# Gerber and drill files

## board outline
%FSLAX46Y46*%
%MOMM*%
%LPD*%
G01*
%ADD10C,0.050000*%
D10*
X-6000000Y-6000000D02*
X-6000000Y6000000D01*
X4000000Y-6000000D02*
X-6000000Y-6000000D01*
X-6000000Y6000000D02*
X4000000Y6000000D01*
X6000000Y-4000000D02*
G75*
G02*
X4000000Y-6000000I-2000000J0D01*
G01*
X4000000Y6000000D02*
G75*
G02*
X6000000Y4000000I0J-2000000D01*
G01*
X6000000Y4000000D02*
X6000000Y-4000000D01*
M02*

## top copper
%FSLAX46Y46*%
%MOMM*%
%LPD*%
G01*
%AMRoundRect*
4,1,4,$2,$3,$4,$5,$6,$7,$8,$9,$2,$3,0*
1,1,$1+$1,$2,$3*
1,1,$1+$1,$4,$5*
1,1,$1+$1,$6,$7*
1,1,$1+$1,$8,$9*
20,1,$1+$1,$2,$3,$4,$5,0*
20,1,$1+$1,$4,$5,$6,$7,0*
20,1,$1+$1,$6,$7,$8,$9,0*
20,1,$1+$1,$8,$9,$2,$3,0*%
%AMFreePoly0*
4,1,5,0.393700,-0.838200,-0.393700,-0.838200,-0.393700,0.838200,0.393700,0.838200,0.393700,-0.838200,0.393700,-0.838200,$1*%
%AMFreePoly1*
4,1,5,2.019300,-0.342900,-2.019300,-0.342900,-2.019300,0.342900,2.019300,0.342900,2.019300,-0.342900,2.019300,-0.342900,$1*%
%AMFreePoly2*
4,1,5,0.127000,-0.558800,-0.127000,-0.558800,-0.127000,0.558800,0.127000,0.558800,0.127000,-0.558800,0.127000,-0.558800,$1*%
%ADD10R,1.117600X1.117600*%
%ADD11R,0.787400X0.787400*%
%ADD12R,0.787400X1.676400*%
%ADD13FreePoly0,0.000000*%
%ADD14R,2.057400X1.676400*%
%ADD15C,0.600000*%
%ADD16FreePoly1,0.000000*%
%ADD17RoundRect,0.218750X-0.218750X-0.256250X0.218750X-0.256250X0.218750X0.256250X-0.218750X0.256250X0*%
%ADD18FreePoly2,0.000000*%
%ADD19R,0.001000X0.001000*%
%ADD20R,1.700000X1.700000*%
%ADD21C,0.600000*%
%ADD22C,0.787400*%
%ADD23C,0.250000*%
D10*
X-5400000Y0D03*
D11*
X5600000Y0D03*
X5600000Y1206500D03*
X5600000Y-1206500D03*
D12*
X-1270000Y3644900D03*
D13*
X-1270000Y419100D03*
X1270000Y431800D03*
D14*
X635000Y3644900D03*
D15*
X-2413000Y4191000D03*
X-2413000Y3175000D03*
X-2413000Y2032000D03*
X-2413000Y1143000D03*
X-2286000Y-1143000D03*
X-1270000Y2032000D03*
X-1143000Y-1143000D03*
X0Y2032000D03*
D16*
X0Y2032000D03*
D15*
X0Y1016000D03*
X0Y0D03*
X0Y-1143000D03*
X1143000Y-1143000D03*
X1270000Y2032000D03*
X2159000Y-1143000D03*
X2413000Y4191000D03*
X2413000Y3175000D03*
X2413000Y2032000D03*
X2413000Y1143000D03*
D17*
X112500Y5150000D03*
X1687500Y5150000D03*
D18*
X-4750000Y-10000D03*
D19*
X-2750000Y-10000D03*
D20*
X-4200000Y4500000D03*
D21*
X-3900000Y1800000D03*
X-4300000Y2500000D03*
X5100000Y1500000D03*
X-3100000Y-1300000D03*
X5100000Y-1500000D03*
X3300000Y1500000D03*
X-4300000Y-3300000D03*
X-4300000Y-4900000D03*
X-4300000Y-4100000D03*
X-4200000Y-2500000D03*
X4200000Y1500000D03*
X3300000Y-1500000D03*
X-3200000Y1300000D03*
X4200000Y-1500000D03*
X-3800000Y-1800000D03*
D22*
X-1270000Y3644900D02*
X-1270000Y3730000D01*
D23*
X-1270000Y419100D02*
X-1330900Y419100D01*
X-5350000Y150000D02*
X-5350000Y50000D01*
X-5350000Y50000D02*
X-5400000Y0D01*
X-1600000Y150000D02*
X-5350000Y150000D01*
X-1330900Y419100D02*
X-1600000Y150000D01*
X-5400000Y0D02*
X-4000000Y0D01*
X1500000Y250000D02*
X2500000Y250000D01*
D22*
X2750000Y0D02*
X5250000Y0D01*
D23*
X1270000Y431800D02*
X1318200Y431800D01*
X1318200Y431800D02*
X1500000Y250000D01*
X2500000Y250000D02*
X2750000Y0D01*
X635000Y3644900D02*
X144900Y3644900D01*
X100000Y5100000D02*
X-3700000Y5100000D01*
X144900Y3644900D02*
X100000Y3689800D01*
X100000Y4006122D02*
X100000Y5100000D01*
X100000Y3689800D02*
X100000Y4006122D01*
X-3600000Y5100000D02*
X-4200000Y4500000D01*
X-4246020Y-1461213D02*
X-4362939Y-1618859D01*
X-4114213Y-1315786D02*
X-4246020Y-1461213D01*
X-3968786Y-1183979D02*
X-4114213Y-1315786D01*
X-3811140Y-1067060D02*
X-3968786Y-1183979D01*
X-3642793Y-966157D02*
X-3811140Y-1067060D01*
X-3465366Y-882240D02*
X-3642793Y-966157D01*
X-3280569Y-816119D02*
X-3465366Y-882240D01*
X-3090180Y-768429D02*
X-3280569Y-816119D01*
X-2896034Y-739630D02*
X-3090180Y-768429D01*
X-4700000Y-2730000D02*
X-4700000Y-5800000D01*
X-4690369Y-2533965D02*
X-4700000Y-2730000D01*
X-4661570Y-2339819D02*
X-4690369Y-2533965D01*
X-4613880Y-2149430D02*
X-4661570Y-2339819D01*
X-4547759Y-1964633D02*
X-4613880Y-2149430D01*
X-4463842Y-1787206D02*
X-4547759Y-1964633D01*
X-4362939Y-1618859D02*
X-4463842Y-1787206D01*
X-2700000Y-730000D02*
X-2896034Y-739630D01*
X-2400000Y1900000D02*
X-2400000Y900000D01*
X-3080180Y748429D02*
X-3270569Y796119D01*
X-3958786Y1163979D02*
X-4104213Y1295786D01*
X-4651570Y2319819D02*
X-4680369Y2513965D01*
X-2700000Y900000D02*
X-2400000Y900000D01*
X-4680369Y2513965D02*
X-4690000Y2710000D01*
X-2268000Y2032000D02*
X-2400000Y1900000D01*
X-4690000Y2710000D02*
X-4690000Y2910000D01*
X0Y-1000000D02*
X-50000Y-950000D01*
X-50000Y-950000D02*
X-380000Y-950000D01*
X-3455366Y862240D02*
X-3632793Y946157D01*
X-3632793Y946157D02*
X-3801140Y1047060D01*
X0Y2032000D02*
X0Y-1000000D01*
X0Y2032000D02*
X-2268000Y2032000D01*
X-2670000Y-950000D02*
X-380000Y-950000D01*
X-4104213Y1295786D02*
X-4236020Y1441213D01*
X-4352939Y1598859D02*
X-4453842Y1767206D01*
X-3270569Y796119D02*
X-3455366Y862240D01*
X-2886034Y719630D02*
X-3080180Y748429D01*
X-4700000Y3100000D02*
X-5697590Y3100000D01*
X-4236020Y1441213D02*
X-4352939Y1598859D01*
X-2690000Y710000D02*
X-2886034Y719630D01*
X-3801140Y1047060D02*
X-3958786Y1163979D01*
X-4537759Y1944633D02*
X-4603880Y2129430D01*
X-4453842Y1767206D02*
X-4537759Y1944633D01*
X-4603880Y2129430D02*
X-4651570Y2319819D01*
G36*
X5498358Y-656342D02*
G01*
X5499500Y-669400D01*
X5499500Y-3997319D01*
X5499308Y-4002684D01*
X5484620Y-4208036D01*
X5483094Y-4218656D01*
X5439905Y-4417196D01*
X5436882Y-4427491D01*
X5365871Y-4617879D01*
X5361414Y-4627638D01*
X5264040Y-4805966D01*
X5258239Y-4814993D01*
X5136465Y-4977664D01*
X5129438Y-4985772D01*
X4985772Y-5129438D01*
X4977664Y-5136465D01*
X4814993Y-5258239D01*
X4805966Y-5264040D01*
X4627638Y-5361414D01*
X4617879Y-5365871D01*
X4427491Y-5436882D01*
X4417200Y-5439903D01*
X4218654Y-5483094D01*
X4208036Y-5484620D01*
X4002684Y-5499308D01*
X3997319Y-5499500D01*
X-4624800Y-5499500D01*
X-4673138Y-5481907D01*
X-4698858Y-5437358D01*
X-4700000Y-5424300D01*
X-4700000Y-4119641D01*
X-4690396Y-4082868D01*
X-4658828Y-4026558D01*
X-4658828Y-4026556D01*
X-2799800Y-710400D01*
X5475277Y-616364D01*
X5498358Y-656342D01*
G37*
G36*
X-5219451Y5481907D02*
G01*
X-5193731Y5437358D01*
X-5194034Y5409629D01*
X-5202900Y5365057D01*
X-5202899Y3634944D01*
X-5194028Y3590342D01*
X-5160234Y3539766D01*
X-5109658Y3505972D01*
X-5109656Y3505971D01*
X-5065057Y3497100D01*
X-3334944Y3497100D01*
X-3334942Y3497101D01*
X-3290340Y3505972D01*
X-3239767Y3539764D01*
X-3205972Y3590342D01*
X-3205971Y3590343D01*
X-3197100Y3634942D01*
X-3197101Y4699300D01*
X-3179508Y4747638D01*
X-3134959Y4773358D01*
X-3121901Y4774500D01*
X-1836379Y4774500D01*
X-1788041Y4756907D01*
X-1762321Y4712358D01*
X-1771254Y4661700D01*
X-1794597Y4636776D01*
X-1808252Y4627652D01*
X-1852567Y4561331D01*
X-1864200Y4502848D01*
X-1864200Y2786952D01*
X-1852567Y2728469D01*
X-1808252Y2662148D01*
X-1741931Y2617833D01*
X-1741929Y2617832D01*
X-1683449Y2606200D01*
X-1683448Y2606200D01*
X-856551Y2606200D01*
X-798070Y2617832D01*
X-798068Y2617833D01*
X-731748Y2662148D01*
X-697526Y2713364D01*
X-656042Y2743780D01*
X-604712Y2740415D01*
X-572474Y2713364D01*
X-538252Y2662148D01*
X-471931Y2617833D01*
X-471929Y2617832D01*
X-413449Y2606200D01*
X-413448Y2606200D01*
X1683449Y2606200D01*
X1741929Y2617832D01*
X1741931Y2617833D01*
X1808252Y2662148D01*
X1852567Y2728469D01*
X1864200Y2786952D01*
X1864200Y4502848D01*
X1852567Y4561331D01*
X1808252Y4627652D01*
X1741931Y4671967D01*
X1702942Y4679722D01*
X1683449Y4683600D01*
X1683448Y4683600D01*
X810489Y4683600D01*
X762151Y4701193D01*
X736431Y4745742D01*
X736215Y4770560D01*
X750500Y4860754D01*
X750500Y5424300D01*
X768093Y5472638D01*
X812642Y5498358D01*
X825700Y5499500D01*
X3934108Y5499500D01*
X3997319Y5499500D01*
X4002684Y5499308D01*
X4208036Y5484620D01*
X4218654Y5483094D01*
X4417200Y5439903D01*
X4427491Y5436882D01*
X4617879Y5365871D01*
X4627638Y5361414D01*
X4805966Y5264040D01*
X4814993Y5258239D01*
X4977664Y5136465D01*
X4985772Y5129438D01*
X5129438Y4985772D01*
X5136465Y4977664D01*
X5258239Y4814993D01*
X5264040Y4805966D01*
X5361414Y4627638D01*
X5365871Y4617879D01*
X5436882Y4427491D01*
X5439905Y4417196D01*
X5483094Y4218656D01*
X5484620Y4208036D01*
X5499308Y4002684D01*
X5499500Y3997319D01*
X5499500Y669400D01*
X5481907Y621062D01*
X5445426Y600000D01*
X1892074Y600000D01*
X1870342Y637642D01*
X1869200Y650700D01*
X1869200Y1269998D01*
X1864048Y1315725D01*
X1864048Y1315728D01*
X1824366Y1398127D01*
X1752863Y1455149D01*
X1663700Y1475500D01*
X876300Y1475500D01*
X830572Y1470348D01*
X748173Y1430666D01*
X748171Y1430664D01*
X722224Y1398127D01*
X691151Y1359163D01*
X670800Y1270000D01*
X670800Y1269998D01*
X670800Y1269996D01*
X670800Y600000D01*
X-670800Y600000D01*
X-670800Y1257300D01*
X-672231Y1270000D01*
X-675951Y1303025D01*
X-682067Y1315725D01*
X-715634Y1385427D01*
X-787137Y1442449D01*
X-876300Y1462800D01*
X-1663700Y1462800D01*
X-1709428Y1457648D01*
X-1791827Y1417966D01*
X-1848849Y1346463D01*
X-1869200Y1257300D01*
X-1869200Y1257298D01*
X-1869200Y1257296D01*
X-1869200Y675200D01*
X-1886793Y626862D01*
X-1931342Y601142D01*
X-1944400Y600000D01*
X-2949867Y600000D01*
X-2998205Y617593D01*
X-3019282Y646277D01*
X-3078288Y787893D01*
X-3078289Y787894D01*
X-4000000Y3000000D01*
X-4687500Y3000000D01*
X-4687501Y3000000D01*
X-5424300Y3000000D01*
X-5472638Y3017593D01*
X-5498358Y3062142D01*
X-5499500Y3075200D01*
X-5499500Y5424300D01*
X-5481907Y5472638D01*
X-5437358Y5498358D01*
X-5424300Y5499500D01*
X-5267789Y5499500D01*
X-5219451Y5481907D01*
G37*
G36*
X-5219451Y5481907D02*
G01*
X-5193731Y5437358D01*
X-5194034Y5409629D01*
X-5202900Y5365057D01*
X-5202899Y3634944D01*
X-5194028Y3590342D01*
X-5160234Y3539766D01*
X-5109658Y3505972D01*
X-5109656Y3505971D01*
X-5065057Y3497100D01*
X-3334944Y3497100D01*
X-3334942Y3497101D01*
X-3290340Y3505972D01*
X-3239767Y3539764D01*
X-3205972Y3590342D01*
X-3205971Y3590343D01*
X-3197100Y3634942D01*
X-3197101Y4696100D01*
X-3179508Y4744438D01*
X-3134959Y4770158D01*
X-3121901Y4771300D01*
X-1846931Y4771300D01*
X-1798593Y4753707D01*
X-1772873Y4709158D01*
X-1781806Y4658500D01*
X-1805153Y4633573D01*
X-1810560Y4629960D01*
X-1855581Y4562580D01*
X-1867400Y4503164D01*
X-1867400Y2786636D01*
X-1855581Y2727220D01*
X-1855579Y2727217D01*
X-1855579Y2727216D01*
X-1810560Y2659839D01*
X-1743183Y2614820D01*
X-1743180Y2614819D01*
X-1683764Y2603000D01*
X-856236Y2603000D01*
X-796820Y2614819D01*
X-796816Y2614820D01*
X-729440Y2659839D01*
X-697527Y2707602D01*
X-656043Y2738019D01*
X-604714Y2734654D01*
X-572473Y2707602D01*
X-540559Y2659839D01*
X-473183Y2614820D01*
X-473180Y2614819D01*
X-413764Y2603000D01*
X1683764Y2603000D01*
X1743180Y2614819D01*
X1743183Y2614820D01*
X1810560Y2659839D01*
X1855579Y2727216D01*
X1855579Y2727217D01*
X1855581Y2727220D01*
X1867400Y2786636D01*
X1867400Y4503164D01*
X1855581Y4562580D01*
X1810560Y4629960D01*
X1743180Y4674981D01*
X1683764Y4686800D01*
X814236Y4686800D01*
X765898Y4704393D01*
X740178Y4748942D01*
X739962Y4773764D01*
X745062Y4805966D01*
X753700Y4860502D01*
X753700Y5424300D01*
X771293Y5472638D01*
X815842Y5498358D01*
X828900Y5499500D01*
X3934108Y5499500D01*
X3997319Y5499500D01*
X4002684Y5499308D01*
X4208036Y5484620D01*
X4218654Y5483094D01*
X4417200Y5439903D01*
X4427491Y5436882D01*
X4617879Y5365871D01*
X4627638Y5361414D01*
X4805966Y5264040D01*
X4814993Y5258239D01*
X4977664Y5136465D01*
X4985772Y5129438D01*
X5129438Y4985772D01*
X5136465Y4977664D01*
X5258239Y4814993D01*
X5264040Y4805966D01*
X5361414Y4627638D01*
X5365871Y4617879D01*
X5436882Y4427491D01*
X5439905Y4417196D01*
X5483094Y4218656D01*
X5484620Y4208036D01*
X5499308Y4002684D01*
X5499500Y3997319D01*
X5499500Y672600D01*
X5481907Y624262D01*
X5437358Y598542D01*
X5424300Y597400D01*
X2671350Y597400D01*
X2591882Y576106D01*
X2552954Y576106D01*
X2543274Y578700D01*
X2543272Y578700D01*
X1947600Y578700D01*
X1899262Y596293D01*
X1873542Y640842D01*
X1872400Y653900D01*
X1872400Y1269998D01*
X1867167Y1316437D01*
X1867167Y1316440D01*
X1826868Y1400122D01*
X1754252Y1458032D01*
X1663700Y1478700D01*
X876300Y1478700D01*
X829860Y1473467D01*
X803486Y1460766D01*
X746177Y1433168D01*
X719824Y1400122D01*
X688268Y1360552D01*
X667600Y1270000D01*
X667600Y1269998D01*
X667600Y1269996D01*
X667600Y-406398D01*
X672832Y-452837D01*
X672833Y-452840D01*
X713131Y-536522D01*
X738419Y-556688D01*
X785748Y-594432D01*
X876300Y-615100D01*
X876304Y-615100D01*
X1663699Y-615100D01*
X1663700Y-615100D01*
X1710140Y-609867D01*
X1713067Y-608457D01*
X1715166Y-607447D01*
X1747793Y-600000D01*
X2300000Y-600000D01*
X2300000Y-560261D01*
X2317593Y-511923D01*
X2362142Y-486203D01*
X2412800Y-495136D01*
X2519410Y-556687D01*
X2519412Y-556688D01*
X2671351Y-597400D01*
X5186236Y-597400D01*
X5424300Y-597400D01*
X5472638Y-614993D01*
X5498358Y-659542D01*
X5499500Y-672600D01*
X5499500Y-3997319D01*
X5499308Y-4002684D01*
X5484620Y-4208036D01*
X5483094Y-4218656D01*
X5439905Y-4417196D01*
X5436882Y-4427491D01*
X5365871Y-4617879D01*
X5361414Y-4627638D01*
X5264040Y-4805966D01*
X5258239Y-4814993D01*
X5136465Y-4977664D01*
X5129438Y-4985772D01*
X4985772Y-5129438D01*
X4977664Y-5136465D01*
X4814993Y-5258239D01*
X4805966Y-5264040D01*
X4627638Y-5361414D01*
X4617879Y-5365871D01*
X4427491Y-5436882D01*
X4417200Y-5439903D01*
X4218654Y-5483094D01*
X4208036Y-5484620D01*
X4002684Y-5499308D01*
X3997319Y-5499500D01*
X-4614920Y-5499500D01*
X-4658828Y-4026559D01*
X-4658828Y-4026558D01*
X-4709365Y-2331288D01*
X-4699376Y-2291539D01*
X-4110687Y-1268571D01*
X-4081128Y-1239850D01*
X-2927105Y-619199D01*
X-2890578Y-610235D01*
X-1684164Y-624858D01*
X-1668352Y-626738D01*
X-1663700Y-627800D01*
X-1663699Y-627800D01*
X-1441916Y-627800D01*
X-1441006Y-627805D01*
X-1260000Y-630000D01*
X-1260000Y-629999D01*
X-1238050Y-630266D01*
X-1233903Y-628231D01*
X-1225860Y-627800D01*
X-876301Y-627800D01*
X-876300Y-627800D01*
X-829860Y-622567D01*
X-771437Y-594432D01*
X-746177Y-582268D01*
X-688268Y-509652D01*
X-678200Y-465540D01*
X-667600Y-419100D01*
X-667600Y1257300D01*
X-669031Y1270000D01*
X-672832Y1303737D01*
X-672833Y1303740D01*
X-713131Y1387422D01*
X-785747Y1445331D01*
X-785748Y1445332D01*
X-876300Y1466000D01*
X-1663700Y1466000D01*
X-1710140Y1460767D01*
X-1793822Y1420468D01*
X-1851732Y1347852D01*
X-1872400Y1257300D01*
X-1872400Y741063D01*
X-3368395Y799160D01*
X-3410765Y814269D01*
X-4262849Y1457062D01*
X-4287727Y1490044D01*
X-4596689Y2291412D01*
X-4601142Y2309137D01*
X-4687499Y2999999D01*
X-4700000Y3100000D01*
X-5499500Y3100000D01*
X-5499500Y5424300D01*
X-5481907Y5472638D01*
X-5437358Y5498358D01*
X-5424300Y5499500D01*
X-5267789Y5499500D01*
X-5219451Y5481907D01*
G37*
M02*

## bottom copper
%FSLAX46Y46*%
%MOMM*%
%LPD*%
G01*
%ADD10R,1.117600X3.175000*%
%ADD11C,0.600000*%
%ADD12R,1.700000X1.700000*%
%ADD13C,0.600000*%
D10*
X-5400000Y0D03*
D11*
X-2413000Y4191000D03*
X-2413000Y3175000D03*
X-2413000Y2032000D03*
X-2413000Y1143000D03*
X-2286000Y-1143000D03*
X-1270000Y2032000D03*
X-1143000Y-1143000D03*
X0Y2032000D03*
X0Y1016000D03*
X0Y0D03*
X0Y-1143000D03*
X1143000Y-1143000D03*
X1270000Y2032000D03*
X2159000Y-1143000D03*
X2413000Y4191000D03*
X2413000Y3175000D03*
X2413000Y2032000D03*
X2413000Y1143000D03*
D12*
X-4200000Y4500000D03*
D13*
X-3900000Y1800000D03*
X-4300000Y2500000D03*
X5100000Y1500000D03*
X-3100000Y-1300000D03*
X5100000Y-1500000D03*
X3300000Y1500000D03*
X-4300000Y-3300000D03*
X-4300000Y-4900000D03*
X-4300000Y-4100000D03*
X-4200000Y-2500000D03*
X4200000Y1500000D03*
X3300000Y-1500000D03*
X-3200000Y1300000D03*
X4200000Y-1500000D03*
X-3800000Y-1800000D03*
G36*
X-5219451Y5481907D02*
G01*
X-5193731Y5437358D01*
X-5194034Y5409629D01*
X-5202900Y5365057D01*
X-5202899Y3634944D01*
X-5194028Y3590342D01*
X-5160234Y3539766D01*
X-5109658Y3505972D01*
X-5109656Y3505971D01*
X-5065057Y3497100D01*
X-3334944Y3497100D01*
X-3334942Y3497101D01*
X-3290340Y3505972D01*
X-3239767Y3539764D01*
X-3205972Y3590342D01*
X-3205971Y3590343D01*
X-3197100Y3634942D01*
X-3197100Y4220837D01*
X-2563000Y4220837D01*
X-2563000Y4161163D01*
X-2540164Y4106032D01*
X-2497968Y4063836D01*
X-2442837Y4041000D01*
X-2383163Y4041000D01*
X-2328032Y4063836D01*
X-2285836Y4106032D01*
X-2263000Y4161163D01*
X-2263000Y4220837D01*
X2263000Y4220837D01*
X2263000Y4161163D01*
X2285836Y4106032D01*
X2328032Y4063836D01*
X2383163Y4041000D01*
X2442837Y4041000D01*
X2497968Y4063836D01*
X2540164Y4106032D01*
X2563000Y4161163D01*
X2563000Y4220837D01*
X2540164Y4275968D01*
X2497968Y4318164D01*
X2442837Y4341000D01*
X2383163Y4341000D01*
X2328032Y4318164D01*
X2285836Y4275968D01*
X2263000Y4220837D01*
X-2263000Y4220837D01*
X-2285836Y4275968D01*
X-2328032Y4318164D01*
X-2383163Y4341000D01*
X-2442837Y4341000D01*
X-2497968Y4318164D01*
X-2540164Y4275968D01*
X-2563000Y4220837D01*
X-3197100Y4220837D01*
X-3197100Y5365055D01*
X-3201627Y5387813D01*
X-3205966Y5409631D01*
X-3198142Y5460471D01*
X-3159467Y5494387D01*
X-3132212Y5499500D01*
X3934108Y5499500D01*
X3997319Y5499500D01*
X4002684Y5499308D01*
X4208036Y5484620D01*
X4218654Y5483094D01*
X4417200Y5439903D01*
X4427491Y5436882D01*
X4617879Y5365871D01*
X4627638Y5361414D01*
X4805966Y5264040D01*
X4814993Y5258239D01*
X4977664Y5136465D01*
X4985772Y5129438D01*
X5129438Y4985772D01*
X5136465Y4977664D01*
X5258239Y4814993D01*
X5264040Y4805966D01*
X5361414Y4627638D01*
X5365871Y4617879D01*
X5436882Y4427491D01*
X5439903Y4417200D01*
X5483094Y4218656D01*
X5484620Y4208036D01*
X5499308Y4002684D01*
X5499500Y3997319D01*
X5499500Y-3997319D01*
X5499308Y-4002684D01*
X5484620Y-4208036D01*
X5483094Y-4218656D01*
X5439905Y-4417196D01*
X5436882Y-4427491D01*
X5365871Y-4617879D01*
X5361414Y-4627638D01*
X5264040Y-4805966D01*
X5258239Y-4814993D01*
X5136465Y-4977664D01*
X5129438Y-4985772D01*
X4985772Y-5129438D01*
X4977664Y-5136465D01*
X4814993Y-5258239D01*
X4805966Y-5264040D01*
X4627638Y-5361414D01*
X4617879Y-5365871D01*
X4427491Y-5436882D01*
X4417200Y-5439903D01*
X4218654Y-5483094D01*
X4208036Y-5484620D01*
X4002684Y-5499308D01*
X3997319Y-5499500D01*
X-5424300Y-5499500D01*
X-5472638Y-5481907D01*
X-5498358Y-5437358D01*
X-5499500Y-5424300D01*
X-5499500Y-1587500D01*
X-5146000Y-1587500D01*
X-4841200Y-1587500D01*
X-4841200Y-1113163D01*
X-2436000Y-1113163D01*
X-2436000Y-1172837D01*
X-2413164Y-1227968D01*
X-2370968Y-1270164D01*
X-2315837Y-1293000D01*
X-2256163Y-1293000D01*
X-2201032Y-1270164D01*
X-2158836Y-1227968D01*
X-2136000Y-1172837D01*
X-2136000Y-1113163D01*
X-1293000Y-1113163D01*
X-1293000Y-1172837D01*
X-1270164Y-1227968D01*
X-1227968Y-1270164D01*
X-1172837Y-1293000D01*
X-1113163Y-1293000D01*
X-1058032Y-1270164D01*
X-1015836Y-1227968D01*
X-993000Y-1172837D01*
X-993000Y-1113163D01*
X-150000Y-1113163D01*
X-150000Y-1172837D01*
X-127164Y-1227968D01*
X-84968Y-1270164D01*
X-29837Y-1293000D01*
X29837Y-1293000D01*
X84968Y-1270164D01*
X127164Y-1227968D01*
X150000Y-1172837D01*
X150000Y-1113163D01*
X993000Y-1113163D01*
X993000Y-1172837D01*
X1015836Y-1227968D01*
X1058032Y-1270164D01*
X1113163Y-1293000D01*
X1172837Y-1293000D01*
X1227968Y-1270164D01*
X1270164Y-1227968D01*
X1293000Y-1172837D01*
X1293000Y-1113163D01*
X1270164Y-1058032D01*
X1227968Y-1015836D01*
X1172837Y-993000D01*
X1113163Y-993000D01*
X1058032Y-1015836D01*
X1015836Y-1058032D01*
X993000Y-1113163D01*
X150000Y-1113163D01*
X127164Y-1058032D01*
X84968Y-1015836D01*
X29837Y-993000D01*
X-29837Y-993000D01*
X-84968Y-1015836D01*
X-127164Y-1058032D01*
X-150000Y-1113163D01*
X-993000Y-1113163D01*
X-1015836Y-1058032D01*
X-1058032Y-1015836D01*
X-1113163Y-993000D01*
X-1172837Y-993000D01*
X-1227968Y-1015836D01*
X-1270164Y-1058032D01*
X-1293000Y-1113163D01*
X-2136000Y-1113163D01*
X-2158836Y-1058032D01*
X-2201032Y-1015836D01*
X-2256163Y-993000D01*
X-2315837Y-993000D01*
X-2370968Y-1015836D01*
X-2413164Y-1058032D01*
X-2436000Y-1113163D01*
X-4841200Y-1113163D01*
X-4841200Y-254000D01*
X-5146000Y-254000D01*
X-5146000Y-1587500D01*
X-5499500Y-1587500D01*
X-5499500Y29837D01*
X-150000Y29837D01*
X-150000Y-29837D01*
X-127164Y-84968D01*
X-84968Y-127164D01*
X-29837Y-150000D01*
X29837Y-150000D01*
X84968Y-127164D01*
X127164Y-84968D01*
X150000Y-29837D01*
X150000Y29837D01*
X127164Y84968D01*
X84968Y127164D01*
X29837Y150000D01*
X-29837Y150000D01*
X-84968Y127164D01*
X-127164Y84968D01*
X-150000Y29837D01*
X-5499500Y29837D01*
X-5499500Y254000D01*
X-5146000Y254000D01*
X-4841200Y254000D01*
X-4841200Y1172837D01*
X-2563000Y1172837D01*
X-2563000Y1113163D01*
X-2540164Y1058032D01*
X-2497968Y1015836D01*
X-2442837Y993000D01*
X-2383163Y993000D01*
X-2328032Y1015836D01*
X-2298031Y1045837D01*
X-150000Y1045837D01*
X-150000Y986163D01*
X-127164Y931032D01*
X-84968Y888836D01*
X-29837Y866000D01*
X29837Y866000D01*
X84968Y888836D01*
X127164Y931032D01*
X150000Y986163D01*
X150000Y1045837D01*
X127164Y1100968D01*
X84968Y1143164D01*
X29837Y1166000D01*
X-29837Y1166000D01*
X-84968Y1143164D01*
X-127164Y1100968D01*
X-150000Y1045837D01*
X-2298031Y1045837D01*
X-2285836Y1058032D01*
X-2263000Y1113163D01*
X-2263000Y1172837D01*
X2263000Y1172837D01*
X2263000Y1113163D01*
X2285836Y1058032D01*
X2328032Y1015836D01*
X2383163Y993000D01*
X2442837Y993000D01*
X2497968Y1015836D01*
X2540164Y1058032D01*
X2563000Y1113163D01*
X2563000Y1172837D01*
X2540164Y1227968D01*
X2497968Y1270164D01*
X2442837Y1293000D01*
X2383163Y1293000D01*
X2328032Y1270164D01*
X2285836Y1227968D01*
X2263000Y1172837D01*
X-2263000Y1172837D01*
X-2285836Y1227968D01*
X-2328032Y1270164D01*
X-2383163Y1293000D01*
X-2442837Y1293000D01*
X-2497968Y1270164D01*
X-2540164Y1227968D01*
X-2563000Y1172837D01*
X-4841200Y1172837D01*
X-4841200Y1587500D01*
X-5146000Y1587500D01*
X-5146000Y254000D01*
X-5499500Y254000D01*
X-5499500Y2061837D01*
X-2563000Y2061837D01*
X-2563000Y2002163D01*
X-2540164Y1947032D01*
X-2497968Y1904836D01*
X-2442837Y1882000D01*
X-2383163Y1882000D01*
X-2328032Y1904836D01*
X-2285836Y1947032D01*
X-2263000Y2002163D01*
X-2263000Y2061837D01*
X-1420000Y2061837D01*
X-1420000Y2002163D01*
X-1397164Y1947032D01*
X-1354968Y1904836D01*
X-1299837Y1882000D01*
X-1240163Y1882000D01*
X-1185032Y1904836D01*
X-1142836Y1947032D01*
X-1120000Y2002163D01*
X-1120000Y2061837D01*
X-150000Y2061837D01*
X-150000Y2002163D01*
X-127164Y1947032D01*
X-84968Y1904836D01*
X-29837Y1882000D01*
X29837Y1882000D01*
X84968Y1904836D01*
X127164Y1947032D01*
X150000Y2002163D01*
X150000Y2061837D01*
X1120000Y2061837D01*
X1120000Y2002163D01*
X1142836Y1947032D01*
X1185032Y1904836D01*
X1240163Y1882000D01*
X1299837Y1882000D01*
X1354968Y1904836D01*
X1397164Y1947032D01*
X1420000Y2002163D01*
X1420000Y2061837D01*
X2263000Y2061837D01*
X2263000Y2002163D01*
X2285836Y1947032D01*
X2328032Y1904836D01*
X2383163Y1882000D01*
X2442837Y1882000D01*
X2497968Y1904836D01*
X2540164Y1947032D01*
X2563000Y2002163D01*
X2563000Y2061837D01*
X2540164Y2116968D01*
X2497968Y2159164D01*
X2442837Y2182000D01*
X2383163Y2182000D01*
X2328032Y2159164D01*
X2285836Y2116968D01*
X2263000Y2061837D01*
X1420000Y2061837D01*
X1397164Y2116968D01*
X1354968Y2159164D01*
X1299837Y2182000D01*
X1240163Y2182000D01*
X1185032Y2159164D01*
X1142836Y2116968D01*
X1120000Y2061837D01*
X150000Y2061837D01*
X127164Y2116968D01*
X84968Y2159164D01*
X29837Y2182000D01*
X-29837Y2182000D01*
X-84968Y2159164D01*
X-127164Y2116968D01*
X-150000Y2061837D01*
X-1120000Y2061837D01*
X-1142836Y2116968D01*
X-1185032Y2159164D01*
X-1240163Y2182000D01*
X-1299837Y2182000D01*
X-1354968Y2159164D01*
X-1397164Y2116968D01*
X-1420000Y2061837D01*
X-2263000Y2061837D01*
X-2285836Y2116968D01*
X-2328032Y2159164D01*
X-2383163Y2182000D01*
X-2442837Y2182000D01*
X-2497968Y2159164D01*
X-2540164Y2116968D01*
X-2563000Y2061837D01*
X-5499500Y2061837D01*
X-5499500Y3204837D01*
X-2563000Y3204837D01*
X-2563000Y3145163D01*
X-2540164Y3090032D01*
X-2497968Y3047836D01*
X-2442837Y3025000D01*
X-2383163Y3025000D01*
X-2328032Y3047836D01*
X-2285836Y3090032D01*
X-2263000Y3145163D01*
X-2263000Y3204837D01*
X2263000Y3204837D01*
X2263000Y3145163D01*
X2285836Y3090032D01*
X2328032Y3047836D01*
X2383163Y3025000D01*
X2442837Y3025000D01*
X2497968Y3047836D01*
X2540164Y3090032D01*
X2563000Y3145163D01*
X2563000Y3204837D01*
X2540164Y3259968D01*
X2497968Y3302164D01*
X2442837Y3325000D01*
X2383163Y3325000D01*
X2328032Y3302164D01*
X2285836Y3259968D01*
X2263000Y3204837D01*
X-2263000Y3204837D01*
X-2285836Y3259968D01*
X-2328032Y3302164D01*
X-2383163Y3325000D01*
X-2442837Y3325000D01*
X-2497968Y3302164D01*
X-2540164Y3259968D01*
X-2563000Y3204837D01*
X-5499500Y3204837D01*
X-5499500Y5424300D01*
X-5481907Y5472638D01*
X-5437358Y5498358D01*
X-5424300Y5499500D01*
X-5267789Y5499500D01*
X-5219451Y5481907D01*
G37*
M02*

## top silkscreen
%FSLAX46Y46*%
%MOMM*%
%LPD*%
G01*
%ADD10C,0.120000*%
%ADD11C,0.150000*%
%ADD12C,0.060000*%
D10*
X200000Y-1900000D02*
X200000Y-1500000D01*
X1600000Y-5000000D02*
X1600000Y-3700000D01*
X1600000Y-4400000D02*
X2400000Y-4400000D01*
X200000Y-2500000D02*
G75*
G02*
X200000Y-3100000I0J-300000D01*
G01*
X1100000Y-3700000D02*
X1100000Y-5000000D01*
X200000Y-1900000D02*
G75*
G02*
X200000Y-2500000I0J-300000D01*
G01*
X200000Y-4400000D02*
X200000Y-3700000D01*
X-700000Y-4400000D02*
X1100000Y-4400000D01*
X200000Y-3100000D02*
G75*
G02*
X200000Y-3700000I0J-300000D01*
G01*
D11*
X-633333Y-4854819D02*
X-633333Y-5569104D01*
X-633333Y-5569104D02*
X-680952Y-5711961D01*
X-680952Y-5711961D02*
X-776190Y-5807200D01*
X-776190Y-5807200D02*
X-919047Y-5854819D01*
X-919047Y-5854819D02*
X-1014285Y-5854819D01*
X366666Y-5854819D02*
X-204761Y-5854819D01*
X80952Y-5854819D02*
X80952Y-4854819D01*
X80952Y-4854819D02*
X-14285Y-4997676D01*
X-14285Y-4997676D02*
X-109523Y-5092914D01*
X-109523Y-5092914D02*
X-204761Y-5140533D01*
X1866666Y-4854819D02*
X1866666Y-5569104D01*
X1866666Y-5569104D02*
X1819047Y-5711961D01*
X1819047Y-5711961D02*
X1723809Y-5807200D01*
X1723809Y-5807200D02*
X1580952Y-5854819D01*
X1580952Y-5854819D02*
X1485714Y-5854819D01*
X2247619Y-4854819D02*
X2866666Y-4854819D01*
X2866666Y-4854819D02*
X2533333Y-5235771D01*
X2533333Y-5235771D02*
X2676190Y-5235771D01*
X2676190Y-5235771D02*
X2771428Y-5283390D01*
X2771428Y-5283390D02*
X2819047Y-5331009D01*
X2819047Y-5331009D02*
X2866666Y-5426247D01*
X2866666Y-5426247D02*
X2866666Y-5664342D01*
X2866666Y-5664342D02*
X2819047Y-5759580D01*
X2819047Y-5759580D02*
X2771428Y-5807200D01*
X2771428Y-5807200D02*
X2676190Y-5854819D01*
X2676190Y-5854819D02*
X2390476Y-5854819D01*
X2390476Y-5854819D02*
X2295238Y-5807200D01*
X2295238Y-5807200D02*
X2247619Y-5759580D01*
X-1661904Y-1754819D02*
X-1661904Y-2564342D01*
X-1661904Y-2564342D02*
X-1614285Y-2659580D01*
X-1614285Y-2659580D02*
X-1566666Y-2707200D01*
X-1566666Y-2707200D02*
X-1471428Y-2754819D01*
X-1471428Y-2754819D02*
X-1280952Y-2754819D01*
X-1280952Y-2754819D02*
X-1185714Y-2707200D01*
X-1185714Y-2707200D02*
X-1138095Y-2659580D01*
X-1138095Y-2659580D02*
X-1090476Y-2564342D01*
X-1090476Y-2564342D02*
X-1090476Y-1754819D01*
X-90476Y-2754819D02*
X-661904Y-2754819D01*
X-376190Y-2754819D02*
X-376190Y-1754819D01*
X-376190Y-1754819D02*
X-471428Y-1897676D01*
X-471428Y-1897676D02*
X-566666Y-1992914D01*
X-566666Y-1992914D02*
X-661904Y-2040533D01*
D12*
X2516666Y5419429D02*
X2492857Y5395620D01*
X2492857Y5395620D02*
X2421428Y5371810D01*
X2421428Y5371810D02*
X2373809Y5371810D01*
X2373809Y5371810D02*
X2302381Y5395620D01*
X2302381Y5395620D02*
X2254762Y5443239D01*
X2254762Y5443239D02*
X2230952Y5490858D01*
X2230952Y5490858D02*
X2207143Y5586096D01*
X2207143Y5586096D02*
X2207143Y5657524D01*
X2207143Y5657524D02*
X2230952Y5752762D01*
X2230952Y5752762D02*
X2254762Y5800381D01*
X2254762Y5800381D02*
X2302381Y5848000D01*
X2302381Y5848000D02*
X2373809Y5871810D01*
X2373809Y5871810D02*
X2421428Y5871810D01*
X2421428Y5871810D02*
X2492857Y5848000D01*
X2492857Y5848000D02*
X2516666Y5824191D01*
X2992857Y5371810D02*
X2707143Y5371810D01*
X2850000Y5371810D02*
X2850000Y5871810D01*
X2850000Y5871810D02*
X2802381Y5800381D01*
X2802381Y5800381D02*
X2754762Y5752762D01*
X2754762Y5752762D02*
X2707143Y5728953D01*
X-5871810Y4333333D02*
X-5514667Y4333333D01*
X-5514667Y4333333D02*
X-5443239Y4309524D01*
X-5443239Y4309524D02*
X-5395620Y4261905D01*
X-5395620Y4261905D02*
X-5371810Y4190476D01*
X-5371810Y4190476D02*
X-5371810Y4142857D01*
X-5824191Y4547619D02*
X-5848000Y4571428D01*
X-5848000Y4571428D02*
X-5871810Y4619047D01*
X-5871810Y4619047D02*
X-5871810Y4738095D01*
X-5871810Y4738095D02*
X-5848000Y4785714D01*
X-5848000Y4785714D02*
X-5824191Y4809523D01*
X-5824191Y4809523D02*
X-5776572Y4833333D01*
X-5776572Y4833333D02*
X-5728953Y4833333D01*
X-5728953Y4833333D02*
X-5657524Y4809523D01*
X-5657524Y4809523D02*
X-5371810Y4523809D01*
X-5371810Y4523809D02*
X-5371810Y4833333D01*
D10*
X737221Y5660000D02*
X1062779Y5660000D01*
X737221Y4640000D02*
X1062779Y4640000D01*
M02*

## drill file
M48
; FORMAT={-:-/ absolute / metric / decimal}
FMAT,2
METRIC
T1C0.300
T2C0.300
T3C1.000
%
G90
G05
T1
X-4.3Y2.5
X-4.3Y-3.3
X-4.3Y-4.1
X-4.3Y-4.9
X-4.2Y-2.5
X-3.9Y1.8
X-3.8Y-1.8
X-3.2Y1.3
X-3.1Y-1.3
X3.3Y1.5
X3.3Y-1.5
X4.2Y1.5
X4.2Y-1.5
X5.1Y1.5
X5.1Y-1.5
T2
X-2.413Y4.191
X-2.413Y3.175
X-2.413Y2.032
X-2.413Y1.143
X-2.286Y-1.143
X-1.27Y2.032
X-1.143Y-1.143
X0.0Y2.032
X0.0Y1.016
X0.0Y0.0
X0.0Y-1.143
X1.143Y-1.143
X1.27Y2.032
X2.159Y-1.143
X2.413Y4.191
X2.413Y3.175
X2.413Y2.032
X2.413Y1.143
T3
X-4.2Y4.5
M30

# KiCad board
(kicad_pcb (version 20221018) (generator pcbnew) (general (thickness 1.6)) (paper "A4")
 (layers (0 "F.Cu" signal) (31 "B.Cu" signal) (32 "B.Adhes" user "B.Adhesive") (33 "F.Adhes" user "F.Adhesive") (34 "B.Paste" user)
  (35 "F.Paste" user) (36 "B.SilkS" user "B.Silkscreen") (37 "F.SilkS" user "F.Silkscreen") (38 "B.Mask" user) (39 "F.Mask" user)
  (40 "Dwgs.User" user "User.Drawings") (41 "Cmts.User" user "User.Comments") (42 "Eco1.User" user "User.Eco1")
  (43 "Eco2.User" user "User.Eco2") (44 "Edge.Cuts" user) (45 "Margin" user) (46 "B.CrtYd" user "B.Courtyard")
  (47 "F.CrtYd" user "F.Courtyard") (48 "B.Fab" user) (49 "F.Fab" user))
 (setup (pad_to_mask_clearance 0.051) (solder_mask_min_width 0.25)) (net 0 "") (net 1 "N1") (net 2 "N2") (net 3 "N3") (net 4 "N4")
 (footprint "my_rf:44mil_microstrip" (layer "F.Cu") (at -5.4 0)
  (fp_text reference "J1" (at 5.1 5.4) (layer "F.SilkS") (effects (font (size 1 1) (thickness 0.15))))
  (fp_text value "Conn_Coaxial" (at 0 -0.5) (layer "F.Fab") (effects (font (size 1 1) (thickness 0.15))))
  (pad "1" smd rect (at 0 0) (size 1.1176 1.1176) (layers "F.Cu" "F.Mask") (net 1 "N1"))
  (pad "2" smd rect (at 0 0) (size 1.1176 3.175) (layers "B.Cu" "B.Mask") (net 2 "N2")))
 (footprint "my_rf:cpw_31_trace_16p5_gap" (layer "F.Cu") (at 5.6 0)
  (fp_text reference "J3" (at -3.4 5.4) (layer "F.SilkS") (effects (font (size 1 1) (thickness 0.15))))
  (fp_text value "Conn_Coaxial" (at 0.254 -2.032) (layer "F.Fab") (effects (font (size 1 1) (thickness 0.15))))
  (pad "1" smd rect (at 0 0) (size 0.7874 0.7874) (layers "F.Cu" "F.Mask") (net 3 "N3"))
  (pad "2" smd rect (at 0 -1.2065) (size 0.7874 0.7874) (layers "F.Cu") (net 2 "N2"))
  (pad "2" smd rect (at 0 1.2065) (size 0.7874 0.7874) (layers "F.Cu") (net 2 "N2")))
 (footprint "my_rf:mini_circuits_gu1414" (layer "F.Cu") (at 0 -2.032)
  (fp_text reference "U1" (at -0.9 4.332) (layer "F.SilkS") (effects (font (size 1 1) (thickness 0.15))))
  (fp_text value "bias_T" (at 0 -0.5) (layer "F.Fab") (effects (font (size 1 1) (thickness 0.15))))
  (pad "" smd rect (at -1.27 -1.6129) (size 0.7874 1.6764) (layers "F.Cu" "F.Paste"))
  (pad "1" smd custom (at -1.27 1.6129) (size 0.7874 1.6764) (layers "F.Cu") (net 1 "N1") (zone_connect 0) (thermal_bridge_angle 45)
   (options (clearance outline) (anchor rect)) (primitives))
  (pad "2" smd custom (at 1.27 1.6002) (size 0.7874 1.6764) (layers "F.Cu") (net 3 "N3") (zone_connect 0) (thermal_bridge_angle 45)
   (options (clearance outline) (anchor rect)) (primitives))
  (pad "3" smd rect (at 0.635 -1.6129) (size 2.0574 1.6764) (layers "F.Cu") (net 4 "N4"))
  (pad "4" thru_hole circle (at -2.413 -2.159) (size 0.6 0.6) (drill 0.3) (layers "*.Cu") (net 2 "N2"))
  (pad "4" thru_hole circle (at -2.413 -1.143) (size 0.6 0.6) (drill 0.3) (layers "*.Cu") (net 2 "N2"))
  (pad "4" thru_hole circle (at -2.413 0) (size 0.6 0.6) (drill 0.3) (layers "*.Cu") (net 2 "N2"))
  (pad "4" thru_hole circle (at -2.413 0.889) (size 0.6 0.6) (drill 0.3) (layers "*.Cu") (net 2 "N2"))
  (pad "4" thru_hole circle (at -2.286 3.175) (size 0.6 0.6) (drill 0.3) (layers "*.Cu") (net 2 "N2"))
  (pad "4" thru_hole circle (at -1.27 0) (size 0.6 0.6) (drill 0.3) (layers "*.Cu") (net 2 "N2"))
  (pad "4" thru_hole circle (at -1.143 3.175) (size 0.6 0.6) (drill 0.3) (layers "*.Cu") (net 2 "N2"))
  (pad "4" thru_hole circle (at 0 0) (size 0.6 0.6) (drill 0.3) (layers "*.Cu") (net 2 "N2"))
  (pad "4" smd custom (at 0 0) (size 4.0386 0.6858) (layers "F.Cu") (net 2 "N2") (zone_connect 2) (thermal_bridge_angle 45)
   (options (clearance outline) (anchor rect)) (primitives))
  (pad "4" thru_hole circle (at 0 1.016) (size 0.6 0.6) (drill 0.3) (layers "*.Cu") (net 2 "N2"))
  (pad "4" thru_hole circle (at 0 2.032) (size 0.6 0.6) (drill 0.3) (layers "*.Cu") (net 2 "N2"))
  (pad "4" thru_hole circle (at 0 3.175) (size 0.6 0.6) (drill 0.3) (layers "*.Cu") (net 2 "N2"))
  (pad "4" thru_hole circle (at 1.143 3.175) (size 0.6 0.6) (drill 0.3) (layers "*.Cu") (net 2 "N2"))
  (pad "4" thru_hole circle (at 1.27 0) (size 0.6 0.6) (drill 0.3) (layers "*.Cu") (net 2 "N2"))
  (pad "4" thru_hole circle (at 2.159 3.175) (size 0.6 0.6) (drill 0.3) (layers "*.Cu") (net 2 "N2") (zone_connect 2))
  (pad "4" thru_hole circle (at 2.413 -2.159) (size 0.6 0.6) (drill 0.3) (layers "*.Cu") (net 2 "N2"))
  (pad "4" thru_hole circle (at 2.413 -1.143) (size 0.6 0.6) (drill 0.3) (layers "*.Cu") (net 2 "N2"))
  (pad "4" thru_hole circle (at 2.413 0) (size 0.6 0.6) (drill 0.3) (layers "*.Cu") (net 2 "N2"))
  (pad "4" thru_hole circle (at 2.413 0.889) (size 0.6 0.6) (drill 0.3) (layers "*.Cu") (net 2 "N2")))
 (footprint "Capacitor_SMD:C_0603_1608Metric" (layer "F.Cu") (at 0.9 -5.15)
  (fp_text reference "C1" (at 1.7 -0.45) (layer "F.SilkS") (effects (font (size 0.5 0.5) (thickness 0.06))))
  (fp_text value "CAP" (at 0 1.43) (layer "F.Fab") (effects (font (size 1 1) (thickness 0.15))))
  (fp_line (start -0.162779 -0.51) (end 0.162779 -0.51) (stroke (width 0.12) (type solid)) (layer "F.SilkS"))
  (fp_line (start -0.162779 0.51) (end 0.162779 0.51) (stroke (width 0.12) (type solid)) (layer "F.SilkS"))
  (pad "1" smd roundrect (at -0.7875 0) (size 0.875 0.95) (layers "F.Cu" "F.Paste" "F.Mask") (roundrect_rratio 0.25) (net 4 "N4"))
  (pad "2" smd roundrect (at 0.7875 0) (size 0.875 0.95) (layers "F.Cu" "F.Paste" "F.Mask") (roundrect_rratio 0.25) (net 2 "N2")))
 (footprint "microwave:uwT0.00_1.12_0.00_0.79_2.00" (layer "F.Cu") (at -4.75 0.01)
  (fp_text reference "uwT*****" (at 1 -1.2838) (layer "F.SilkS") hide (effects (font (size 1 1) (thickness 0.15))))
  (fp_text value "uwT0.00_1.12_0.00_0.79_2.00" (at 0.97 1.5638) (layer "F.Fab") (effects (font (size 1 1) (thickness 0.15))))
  (pad "1" smd custom (at 0 0) (size 0.254 1.1176) (layers "F.Cu") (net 1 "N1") (zone_connect 0) (thermal_bridge_angle 45)
   (options (clearance outline) (anchor rect)) (primitives))
  (pad "1" smd rect (at 2 0) (size 0.001 0.001) (layers "F.Cu")))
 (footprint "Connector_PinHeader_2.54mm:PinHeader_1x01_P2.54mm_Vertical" (layer "B.Cu") (at -4.2 -4.5)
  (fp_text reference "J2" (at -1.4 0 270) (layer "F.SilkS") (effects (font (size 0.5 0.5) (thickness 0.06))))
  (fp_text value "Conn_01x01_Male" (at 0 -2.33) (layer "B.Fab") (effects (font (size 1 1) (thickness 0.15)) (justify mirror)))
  (pad "1" thru_hole rect (at 0 0) (size 1.7 1.7) (drill 1) (layers "*.Cu" "*.Mask") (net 4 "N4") (clearance 0.1524)))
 (gr_line (start 0.2 1.9) (end 0.2 1.5) (stroke (width 0.12) (type solid)) (layer "F.SilkS"))
 (gr_line (start 1.6 5) (end 1.6 3.7) (stroke (width 0.12) (type solid)) (layer "F.SilkS"))
 (gr_line (start 1.6 4.4) (end 2.4 4.4) (stroke (width 0.12) (type solid)) (layer "F.SilkS"))
 (gr_arc (start 0.2 2.5) (mid 0.5 2.8) (end 0.2 3.1) (stroke (width 0.12) (type solid)) (layer "F.SilkS"))
 (gr_line (start 1.1 3.7) (end 1.1 5) (stroke (width 0.12) (type solid)) (layer "F.SilkS"))
 (gr_arc (start 0.2 1.9) (mid 0.5 2.2) (end 0.2 2.5) (stroke (width 0.12) (type solid)) (layer "F.SilkS"))
 (gr_line (start 0.2 4.4) (end 0.2 3.7) (stroke (width 0.12) (type solid)) (layer "F.SilkS"))
 (gr_line (start -0.7 4.4) (end 1.1 4.4) (stroke (width 0.12) (type solid)) (layer "F.SilkS"))
 (gr_arc (start 0.2 3.1) (mid 0.5 3.4) (end 0.2 3.7) (stroke (width 0.12) (type solid)) (layer "F.SilkS"))
 (gr_line (start -6 6) (end -6 -6) (stroke (width 0.05) (type solid)) (layer "Edge.Cuts"))
 (gr_line (start 4 6) (end -6 6) (stroke (width 0.05) (type solid)) (layer "Edge.Cuts"))
 (gr_line (start -6 -6) (end 4 -6) (stroke (width 0.05) (type solid)) (layer "Edge.Cuts"))
 (gr_arc (start 6 4) (mid 5.414214 5.414214) (end 4 6) (stroke (width 0.05) (type solid)) (layer "Edge.Cuts"))
 (gr_arc (start 4 -6) (mid 5.414214 -5.414214) (end 6 -4) (stroke (width 0.05) (type solid)) (layer "Edge.Cuts"))
 (gr_line (start 6 -4) (end 6 4) (stroke (width 0.05) (type solid)) (layer "Edge.Cuts"))
 (segment (start -1.27 -3.6449) (end -1.27 -3.73) (width 0.7874) (layer "F.Cu") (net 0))
 (segment (start -1.27 -0.4191) (end -1.3309 -0.4191) (width 0.25) (layer "F.Cu") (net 1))
 (segment (start -5.35 -0.15) (end -5.35 -0.05) (width 0.25) (layer "F.Cu") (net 1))
 (segment (start -5.35 -0.05) (end -5.4 0) (width 0.25) (layer "F.Cu") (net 1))
 (segment (start -1.6 -0.15) (end -5.35 -0.15) (width 0.25) (layer "F.Cu") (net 1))
 (segment (start -1.3309 -0.4191) (end -1.6 -0.15) (width 0.25) (layer "F.Cu") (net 1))
 (segment (start -5.4 0) (end -4 0) (width 0.25) (layer "F.Cu") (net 1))
 (segment (start 1.5 -0.25) (end 2.5 -0.25) (width 0.25) (layer "F.Cu") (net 3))
 (segment (start 2.75 0) (end 5.25 0) (width 0.7874) (layer "F.Cu") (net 3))
 (segment (start 1.27 -0.4318) (end 1.3182 -0.4318) (width 0.25) (layer "F.Cu") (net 3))
 (segment (start 1.3182 -0.4318) (end 1.5 -0.25) (width 0.25) (layer "F.Cu") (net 3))
 (segment (start 2.5 -0.25) (end 2.75 0) (width 0.25) (layer "F.Cu") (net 3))
 (segment (start 0.635 -3.6449) (end 0.1449 -3.6449) (width 0.25) (layer "F.Cu") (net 4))
 (segment (start 0.1 -5.1) (end -3.7 -5.1) (width 0.25) (layer "F.Cu") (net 4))
 (segment (start 0.1449 -3.6449) (end 0.1 -3.6898) (width 0.25) (layer "F.Cu") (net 4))
 (segment (start 0.1 -4.006122) (end 0.1 -5.1) (width 0.25) (layer "F.Cu") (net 4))
 (segment (start 0.1 -3.6898) (end 0.1 -4.006122) (width 0.25) (layer "F.Cu") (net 4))
 (segment (start -3.6 -5.1) (end -4.2 -4.5) (width 0.25) (layer "F.Cu") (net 4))
 (segment (start -4.24602 1.461213) (end -4.362939 1.618859) (width 0.25) (layer "F.Cu") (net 2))
 (segment (start -4.114213 1.315786) (end -4.24602 1.461213) (width 0.25) (layer "F.Cu") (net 2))
 (segment (start -3.968786 1.183979) (end -4.114213 1.315786) (width 0.25) (layer "F.Cu") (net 2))
 (segment (start -3.81114 1.06706) (end -3.968786 1.183979) (width 0.25) (layer "F.Cu") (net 2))
 (segment (start -3.642793 0.966157) (end -3.81114 1.06706) (width 0.25) (layer "F.Cu") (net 2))
 (segment (start -3.465366 0.88224) (end -3.642793 0.966157) (width 0.25) (layer "F.Cu") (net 2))
 (segment (start -3.280569 0.816119) (end -3.465366 0.88224) (width 0.25) (layer "F.Cu") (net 2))
 (segment (start -3.09018 0.768429) (end -3.280569 0.816119) (width 0.25) (layer "F.Cu") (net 2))
 (segment (start -2.896034 0.73963) (end -3.09018 0.768429) (width 0.25) (layer "F.Cu") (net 2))
 (segment (start -4.7 2.73) (end -4.7 5.8) (width 0.25) (layer "F.Cu") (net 2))
 (segment (start -4.690369 2.533965) (end -4.7 2.73) (width 0.25) (layer "F.Cu") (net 2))
 (segment (start -4.66157 2.339819) (end -4.690369 2.533965) (width 0.25) (layer "F.Cu") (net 2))
 (segment (start -4.61388 2.14943) (end -4.66157 2.339819) (width 0.25) (layer "F.Cu") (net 2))
 (segment (start -4.547759 1.964633) (end -4.61388 2.14943) (width 0.25) (layer "F.Cu") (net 2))
 (segment (start -4.463842 1.787206) (end -4.547759 1.964633) (width 0.25) (layer "F.Cu") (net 2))
 (segment (start -4.362939 1.618859) (end -4.463842 1.787206) (width 0.25) (layer "F.Cu") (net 2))
 (segment (start -2.7 0.73) (end -2.896034 0.73963) (width 0.25) (layer "F.Cu") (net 2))
 (segment (start -2.4 -1.9) (end -2.4 -0.9) (width 0.25) (layer "F.Cu") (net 2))
 (segment (start -3.08018 -0.748429) (end -3.270569 -0.796119) (width 0.25) (layer "F.Cu") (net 2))
 (segment (start -3.958786 -1.163979) (end -4.104213 -1.295786) (width 0.25) (layer "F.Cu") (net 2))
 (segment (start -4.65157 -2.319819) (end -4.680369 -2.513965) (width 0.25) (layer "F.Cu") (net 2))
 (segment (start -2.7 -0.9) (end -2.4 -0.9) (width 0.25) (layer "F.Cu") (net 2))
 (segment (start -4.680369 -2.513965) (end -4.69 -2.71) (width 0.25) (layer "F.Cu") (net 2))
 (segment (start -2.268 -2.032) (end -2.4 -1.9) (width 0.25) (layer "F.Cu") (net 2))
 (segment (start -4.69 -2.71) (end -4.69 -2.91) (width 0.25) (layer "F.Cu") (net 2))
 (segment (start 0 1) (end -0.05 0.95) (width 0.25) (layer "F.Cu") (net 2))
 (segment (start -0.05 0.95) (end -0.38 0.95) (width 0.25) (layer "F.Cu") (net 2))
 (segment (start -3.455366 -0.86224) (end -3.632793 -0.946157) (width 0.25) (layer "F.Cu") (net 2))
 (segment (start -3.632793 -0.946157) (end -3.80114 -1.04706) (width 0.25) (layer "F.Cu") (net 2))
 (segment (start 0 -2.032) (end 0 1) (width 0.25) (layer "F.Cu") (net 2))
 (segment (start 0 -2.032) (end -2.268 -2.032) (width 0.25) (layer "F.Cu") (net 2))
 (segment (start -2.67 0.95) (end -0.38 0.95) (width 0.25) (layer "F.Cu") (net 2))
 (segment (start -4.104213 -1.295786) (end -4.23602 -1.441213) (width 0.25) (layer "F.Cu") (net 2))
 (segment (start -4.352939 -1.598859) (end -4.453842 -1.767206) (width 0.25) (layer "F.Cu") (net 2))
 (segment (start -3.270569 -0.796119) (end -3.455366 -0.86224) (width 0.25) (layer "F.Cu") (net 2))
 (segment (start -2.886034 -0.71963) (end -3.08018 -0.748429) (width 0.25) (layer "F.Cu") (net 2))
 (segment (start -4.7 -3.1) (end -5.69759 -3.1) (width 0.25) (layer "F.Cu") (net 2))
 (segment (start -4.23602 -1.441213) (end -4.352939 -1.598859) (width 0.25) (layer "F.Cu") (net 2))
 (segment (start -2.69 -0.71) (end -2.886034 -0.71963) (width 0.25) (layer "F.Cu") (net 2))
 (segment (start -3.80114 -1.04706) (end -3.958786 -1.163979) (width 0.25) (layer "F.Cu") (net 2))
 (segment (start -4.537759 -1.944633) (end -4.60388 -2.12943) (width 0.25) (layer "F.Cu") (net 2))
 (segment (start -4.453842 -1.767206) (end -4.537759 -1.944633) (width 0.25) (layer "F.Cu") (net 2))
 (segment (start -4.60388 -2.12943) (end -4.65157 -2.319819) (width 0.25) (layer "F.Cu") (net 2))
 (via (at -3.9 -1.8) (size 0.6) (drill 0.3) (layers "F.Cu" "B.Cu") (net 2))
 (via (at -4.3 -2.5) (size 0.6) (drill 0.3) (layers "F.Cu" "B.Cu") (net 2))
 (via (at 5.1 -1.5) (size 0.6) (drill 0.3) (layers "F.Cu" "B.Cu") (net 2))
 (via (at -3.1 1.3) (size 0.6) (drill 0.3) (layers "F.Cu" "B.Cu") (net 2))
 (via (at 5.1 1.5) (size 0.6) (drill 0.3) (layers "F.Cu" "B.Cu") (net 2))
 (via (at 3.3 -1.5) (size 0.6) (drill 0.3) (layers "F.Cu" "B.Cu") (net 2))
 (via (at -4.3 3.3) (size 0.6) (drill 0.3) (layers "F.Cu" "B.Cu") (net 2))
 (via (at -4.3 4.9) (size 0.6) (drill 0.3) (layers "F.Cu" "B.Cu") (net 2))
 (via (at -4.3 4.1) (size 0.6) (drill 0.3) (layers "F.Cu" "B.Cu") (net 2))
 (via (at -4.2 2.5) (size 0.6) (drill 0.3) (layers "F.Cu" "B.Cu") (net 2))
 (via (at 4.2 -1.5) (size 0.6) (drill 0.3) (layers "F.Cu" "B.Cu") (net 2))
 (via (at 3.3 1.5) (size 0.6) (drill 0.3) (layers "F.Cu" "B.Cu") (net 2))
 (via (at -3.2 -1.3) (size 0.6) (drill 0.3) (layers "F.Cu" "B.Cu") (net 2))
 (via (at 4.2 1.5) (size 0.6) (drill 0.3) (layers "F.Cu" "B.Cu") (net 2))
 (via (at -3.8 1.8) (size 0.6) (drill 0.3) (layers "F.Cu" "B.Cu") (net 2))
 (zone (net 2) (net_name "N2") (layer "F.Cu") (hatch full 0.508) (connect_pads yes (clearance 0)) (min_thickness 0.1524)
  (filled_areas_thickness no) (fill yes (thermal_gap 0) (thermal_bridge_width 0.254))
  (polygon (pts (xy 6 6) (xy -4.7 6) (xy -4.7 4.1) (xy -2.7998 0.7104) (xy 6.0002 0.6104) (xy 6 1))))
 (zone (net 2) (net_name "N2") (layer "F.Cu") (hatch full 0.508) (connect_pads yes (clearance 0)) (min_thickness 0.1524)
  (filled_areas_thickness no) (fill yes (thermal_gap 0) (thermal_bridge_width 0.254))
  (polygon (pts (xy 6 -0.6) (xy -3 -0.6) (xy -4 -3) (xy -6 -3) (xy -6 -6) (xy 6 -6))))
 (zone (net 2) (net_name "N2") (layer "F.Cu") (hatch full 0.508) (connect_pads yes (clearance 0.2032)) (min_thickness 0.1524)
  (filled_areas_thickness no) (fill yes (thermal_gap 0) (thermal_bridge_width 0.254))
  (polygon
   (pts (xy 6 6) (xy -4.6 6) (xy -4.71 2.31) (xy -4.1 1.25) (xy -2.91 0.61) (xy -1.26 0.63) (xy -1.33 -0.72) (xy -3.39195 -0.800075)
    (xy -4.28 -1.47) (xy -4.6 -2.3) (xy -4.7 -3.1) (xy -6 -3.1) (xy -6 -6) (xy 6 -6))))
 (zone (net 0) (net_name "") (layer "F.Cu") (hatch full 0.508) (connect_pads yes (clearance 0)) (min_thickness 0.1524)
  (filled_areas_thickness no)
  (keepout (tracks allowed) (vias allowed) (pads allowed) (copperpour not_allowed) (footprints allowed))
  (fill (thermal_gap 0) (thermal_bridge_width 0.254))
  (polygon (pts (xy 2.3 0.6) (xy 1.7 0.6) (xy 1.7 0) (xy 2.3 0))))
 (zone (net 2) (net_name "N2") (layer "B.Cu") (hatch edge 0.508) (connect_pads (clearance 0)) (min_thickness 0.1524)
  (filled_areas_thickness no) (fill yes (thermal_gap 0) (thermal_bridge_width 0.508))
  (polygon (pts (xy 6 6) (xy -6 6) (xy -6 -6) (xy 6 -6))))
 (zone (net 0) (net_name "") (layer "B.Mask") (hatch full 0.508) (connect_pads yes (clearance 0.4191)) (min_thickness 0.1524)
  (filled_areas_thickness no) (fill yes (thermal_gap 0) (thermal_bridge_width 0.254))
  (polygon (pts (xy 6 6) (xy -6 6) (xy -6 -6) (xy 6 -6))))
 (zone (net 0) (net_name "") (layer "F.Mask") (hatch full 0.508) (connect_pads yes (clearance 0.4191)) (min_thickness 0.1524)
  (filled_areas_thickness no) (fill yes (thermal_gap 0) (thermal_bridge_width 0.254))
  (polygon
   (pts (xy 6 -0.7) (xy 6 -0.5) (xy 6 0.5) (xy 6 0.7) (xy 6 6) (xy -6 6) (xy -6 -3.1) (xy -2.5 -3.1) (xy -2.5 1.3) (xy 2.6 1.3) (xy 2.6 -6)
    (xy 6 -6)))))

